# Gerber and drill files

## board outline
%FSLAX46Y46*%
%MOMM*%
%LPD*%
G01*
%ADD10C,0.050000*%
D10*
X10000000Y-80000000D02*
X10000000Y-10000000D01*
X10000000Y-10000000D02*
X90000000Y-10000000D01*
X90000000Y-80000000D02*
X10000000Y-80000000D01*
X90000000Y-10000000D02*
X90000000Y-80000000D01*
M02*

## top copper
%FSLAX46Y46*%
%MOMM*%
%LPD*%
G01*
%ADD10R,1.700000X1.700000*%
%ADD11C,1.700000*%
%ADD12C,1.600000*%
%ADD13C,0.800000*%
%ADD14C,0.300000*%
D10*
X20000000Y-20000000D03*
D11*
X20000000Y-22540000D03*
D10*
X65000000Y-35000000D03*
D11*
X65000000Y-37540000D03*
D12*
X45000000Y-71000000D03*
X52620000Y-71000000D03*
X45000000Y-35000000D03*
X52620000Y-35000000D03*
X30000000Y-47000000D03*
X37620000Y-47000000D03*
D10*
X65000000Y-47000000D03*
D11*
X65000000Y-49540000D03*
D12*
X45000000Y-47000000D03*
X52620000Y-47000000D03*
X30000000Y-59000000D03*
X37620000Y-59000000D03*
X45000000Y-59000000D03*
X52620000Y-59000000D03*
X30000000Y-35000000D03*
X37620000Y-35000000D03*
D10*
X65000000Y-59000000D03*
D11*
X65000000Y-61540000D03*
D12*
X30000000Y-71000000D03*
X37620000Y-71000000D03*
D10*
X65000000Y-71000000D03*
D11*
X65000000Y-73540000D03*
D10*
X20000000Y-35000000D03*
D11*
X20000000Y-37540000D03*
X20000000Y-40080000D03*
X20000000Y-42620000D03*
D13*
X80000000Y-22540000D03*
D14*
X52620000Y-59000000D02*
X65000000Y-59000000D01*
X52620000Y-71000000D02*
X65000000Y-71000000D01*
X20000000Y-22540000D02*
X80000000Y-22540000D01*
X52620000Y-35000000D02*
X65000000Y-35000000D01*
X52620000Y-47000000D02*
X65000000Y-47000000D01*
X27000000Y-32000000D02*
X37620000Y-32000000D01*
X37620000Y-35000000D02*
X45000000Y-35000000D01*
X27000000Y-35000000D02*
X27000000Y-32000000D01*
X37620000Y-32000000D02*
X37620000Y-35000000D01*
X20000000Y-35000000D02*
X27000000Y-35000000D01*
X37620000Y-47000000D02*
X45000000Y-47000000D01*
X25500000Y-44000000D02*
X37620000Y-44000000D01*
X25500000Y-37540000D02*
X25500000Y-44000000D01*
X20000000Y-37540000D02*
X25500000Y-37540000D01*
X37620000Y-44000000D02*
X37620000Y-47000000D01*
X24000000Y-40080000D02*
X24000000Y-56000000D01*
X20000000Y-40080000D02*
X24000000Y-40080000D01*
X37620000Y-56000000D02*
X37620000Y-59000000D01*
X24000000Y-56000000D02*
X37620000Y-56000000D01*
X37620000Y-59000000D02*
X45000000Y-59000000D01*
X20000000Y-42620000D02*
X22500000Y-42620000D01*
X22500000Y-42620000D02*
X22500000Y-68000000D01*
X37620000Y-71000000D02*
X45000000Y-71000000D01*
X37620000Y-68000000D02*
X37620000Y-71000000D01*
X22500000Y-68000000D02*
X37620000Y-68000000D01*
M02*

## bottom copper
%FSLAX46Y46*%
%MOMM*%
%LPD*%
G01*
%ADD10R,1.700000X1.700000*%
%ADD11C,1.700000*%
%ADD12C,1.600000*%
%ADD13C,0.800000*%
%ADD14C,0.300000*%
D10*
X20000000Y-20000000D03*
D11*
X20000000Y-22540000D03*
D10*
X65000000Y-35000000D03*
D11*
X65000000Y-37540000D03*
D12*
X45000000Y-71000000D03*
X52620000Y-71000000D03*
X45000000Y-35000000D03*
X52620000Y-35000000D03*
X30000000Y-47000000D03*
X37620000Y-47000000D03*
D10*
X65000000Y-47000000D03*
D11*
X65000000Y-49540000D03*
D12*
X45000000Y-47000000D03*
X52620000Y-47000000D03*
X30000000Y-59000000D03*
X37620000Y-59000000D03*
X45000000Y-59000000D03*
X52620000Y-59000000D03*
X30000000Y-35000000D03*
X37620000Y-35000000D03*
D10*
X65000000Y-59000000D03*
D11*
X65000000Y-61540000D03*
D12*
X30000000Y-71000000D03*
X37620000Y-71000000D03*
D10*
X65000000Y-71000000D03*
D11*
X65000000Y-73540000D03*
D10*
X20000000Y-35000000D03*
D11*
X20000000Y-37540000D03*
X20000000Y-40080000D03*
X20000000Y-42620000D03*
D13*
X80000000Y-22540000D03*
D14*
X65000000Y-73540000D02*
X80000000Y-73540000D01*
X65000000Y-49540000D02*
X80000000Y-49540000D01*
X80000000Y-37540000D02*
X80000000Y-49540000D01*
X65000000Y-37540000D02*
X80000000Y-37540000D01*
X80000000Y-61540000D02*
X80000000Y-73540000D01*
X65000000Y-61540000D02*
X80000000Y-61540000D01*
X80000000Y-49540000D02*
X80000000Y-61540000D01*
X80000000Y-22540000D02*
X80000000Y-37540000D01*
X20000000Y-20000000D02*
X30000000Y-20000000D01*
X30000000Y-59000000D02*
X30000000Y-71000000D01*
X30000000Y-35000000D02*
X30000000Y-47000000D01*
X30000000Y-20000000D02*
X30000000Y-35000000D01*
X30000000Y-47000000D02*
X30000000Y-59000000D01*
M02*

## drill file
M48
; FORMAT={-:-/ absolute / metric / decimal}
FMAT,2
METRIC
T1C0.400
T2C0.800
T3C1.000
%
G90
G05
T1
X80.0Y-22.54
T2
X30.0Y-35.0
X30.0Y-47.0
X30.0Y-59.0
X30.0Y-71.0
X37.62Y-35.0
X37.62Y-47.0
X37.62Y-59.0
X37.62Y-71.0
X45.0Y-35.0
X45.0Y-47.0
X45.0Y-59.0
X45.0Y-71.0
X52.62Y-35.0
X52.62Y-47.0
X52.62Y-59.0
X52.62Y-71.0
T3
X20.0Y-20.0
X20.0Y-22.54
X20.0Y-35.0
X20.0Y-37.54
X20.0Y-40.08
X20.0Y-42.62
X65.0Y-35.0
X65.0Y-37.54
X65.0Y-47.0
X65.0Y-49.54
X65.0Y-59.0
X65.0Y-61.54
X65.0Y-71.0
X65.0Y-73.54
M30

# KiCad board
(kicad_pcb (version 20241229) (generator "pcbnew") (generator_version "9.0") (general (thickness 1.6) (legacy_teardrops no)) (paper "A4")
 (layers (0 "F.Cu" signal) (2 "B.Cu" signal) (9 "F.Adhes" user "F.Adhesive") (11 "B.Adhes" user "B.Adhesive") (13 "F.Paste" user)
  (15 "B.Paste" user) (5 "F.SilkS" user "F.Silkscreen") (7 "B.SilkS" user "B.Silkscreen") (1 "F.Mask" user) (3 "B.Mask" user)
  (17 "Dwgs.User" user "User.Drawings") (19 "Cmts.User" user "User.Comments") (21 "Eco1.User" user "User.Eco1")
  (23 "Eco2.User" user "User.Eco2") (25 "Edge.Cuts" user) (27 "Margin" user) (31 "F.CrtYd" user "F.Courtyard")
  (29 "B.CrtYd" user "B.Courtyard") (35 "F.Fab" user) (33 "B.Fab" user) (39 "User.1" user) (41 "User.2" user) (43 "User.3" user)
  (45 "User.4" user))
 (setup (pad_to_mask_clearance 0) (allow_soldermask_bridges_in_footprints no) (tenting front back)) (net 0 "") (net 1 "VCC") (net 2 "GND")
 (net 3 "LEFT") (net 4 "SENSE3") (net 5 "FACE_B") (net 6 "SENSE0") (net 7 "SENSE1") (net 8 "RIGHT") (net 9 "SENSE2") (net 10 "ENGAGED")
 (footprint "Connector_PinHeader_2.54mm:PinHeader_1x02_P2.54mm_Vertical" (layer "F.Cu") (at 20 20)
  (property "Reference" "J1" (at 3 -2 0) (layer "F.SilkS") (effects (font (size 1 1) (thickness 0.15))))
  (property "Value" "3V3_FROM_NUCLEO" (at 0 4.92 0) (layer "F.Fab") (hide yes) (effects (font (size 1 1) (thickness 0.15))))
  (pad "1" thru_hole rect (at 0 0) (size 1.7 1.7) (drill 1) (layers "*.Cu" "*.Mask") (remove_unused_layers no) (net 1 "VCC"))
  (pad "2" thru_hole circle (at 0 2.54) (size 1.7 1.7) (drill 1) (layers "*.Cu" "*.Mask") (remove_unused_layers no) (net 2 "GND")))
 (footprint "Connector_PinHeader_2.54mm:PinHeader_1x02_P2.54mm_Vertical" (layer "F.Cu") (at 65 35)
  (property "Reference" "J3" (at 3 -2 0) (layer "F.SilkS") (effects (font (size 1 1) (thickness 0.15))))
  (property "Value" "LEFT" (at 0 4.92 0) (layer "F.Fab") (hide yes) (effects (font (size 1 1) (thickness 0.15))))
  (pad "1" thru_hole rect (at 0 0) (size 1.7 1.7) (drill 1) (layers "*.Cu" "*.Mask") (remove_unused_layers no) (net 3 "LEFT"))
  (pad "2" thru_hole circle (at 0 2.54) (size 1.7 1.7) (drill 1) (layers "*.Cu" "*.Mask") (remove_unused_layers no) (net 2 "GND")))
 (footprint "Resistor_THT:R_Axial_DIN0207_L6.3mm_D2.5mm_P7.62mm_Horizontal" (layer "F.Cu") (at 45 71)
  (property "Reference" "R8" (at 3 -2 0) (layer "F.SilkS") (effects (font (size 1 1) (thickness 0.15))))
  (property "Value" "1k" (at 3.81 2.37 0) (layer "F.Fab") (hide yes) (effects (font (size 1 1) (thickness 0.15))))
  (pad "1" thru_hole circle (at 0 0) (size 1.6 1.6) (drill 0.8) (layers "*.Cu" "*.Mask") (remove_unused_layers no) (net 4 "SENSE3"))
  (pad "2" thru_hole circle (at 7.62 0) (size 1.6 1.6) (drill 0.8) (layers "*.Cu" "*.Mask") (remove_unused_layers no) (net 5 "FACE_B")))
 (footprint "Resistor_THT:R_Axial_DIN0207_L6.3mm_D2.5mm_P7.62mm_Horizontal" (layer "F.Cu") (at 45 35)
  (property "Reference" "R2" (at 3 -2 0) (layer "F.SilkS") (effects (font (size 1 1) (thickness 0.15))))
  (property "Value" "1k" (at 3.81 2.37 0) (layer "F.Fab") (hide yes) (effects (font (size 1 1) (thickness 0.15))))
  (pad "1" thru_hole circle (at 0 0) (size 1.6 1.6) (drill 0.8) (layers "*.Cu" "*.Mask") (remove_unused_layers no) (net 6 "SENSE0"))
  (pad "2" thru_hole circle (at 7.62 0) (size 1.6 1.6) (drill 0.8) (layers "*.Cu" "*.Mask") (remove_unused_layers no) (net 3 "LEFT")))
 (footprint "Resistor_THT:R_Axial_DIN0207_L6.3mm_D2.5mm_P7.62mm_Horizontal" (layer "F.Cu") (at 30 47)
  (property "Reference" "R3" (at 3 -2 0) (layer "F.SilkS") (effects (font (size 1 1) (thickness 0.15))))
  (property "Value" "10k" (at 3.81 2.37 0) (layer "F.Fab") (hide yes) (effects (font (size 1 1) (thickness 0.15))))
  (pad "1" thru_hole circle (at 0 0) (size 1.6 1.6) (drill 0.8) (layers "*.Cu" "*.Mask") (remove_unused_layers no) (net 1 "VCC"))
  (pad "2" thru_hole circle (at 7.62 0) (size 1.6 1.6) (drill 0.8) (layers "*.Cu" "*.Mask") (remove_unused_layers no) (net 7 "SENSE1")))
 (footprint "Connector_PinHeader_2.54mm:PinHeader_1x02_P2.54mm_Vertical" (layer "F.Cu") (at 65 47)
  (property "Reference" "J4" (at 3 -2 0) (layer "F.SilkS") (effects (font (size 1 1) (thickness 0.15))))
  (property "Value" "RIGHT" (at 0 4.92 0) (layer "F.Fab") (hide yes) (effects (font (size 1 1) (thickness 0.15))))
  (pad "1" thru_hole rect (at 0 0) (size 1.7 1.7) (drill 1) (layers "*.Cu" "*.Mask") (remove_unused_layers no) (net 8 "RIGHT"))
  (pad "2" thru_hole circle (at 0 2.54) (size 1.7 1.7) (drill 1) (layers "*.Cu" "*.Mask") (remove_unused_layers no) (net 2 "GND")))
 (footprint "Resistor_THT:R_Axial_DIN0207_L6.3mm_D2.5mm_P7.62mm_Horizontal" (layer "F.Cu") (at 45 47)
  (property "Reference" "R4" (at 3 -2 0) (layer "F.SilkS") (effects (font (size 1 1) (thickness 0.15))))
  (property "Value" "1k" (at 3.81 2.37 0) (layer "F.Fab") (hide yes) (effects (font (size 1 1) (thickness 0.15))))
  (pad "1" thru_hole circle (at 0 0) (size 1.6 1.6) (drill 0.8) (layers "*.Cu" "*.Mask") (remove_unused_layers no) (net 7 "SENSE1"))
  (pad "2" thru_hole circle (at 7.62 0) (size 1.6 1.6) (drill 0.8) (layers "*.Cu" "*.Mask") (remove_unused_layers no) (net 8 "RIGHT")))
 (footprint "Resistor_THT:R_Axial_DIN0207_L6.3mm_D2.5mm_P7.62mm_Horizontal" (layer "F.Cu") (at 30 59)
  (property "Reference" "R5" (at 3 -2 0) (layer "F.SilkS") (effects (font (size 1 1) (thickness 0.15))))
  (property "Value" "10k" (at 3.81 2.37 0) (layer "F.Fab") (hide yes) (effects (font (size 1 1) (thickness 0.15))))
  (pad "1" thru_hole circle (at 0 0) (size 1.6 1.6) (drill 0.8) (layers "*.Cu" "*.Mask") (remove_unused_layers no) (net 1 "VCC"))
  (pad "2" thru_hole circle (at 7.62 0) (size 1.6 1.6) (drill 0.8) (layers "*.Cu" "*.Mask") (remove_unused_layers no) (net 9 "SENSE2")))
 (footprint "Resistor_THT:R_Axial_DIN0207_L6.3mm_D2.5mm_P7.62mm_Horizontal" (layer "F.Cu") (at 45 59)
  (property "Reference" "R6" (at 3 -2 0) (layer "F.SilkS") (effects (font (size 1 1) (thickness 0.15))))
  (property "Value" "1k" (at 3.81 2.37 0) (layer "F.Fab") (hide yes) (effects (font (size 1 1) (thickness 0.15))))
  (pad "1" thru_hole circle (at 0 0) (size 1.6 1.6) (drill 0.8) (layers "*.Cu" "*.Mask") (remove_unused_layers no) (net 9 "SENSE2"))
  (pad "2" thru_hole circle (at 7.62 0) (size 1.6 1.6) (drill 0.8) (layers "*.Cu" "*.Mask") (remove_unused_layers no) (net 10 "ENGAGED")))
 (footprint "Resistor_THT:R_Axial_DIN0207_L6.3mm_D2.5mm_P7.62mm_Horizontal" (layer "F.Cu") (at 30 35)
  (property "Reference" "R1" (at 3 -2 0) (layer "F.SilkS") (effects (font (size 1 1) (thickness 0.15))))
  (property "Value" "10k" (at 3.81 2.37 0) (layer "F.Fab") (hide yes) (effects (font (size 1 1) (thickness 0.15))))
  (pad "1" thru_hole circle (at 0 0) (size 1.6 1.6) (drill 0.8) (layers "*.Cu" "*.Mask") (remove_unused_layers no) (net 1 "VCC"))
  (pad "2" thru_hole circle (at 7.62 0) (size 1.6 1.6) (drill 0.8) (layers "*.Cu" "*.Mask") (remove_unused_layers no) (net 6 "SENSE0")))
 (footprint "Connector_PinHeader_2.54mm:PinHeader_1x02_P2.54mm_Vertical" (layer "F.Cu") (at 65 59)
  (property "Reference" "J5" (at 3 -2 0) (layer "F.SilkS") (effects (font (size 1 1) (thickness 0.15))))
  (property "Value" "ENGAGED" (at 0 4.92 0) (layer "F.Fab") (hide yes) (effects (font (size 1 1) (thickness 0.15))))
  (pad "1" thru_hole rect (at 0 0) (size 1.7 1.7) (drill 1) (layers "*.Cu" "*.Mask") (remove_unused_layers no) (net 10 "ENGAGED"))
  (pad "2" thru_hole circle (at 0 2.54) (size 1.7 1.7) (drill 1) (layers "*.Cu" "*.Mask") (remove_unused_layers no) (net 2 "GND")))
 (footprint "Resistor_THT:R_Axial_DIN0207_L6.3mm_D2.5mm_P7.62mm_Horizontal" (layer "F.Cu") (at 30 71)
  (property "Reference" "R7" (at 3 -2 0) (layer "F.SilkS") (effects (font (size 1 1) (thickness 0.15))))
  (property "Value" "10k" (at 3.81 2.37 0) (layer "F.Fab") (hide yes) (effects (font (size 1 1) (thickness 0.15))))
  (pad "1" thru_hole circle (at 0 0) (size 1.6 1.6) (drill 0.8) (layers "*.Cu" "*.Mask") (remove_unused_layers no) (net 1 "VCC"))
  (pad "2" thru_hole circle (at 7.62 0) (size 1.6 1.6) (drill 0.8) (layers "*.Cu" "*.Mask") (remove_unused_layers no) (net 4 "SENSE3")))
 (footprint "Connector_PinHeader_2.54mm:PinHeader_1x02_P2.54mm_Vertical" (layer "F.Cu") (at 65 71)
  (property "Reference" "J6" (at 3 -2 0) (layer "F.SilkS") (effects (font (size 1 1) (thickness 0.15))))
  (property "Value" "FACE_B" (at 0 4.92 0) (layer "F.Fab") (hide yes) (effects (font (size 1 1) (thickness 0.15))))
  (pad "1" thru_hole rect (at 0 0) (size 1.7 1.7) (drill 1) (layers "*.Cu" "*.Mask") (remove_unused_layers no) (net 5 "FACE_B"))
  (pad "2" thru_hole circle (at 0 2.54) (size 1.7 1.7) (drill 1) (layers "*.Cu" "*.Mask") (remove_unused_layers no) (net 2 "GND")))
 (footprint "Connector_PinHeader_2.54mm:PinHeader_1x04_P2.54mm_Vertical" (layer "F.Cu") (at 20 35)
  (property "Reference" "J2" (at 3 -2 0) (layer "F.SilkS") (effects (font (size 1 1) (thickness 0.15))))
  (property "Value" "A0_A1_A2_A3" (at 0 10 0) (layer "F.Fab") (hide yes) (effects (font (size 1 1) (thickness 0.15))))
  (pad "1" thru_hole rect (at 0 0) (size 1.7 1.7) (drill 1) (layers "*.Cu" "*.Mask") (remove_unused_layers no) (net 6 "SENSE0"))
  (pad "2" thru_hole circle (at 0 2.54) (size 1.7 1.7) (drill 1) (layers "*.Cu" "*.Mask") (remove_unused_layers no) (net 7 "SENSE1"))
  (pad "3" thru_hole circle (at 0 5.08) (size 1.7 1.7) (drill 1) (layers "*.Cu" "*.Mask") (remove_unused_layers no) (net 9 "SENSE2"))
  (pad "4" thru_hole circle (at 0 7.62) (size 1.7 1.7) (drill 1) (layers "*.Cu" "*.Mask") (remove_unused_layers no) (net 4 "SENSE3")))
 (gr_line (start 10 80) (end 10 10) (stroke (width 0.05) (type default)) (layer "Edge.Cuts"))
 (gr_line (start 10 10) (end 90 10) (stroke (width 0.05) (type default)) (layer "Edge.Cuts"))
 (gr_line (start 90 80) (end 10 80) (stroke (width 0.05) (type default)) (layer "Edge.Cuts"))
 (gr_line (start 90 10) (end 90 80) (stroke (width 0.05) (type default)) (layer "Edge.Cuts"))
 (segment (start 52.62 59) (end 65 59) (width 0.3) (layer "F.Cu") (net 10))
 (segment (start 52.62 71) (end 65 71) (width 0.3) (layer "F.Cu") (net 5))
 (segment (start 20 22.54) (end 80 22.54) (width 0.3) (layer "F.Cu") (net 2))
 (via (at 80 22.54) (size 0.8) (drill 0.4) (layers "F.Cu" "B.Cu") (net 2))
 (segment (start 65 73.54) (end 80 73.54) (width 0.3) (layer "B.Cu") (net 2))
 (segment (start 65 49.54) (end 80 49.54) (width 0.3) (layer "B.Cu") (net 2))
 (segment (start 80 37.54) (end 80 49.54) (width 0.3) (layer "B.Cu") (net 2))
 (segment (start 65 37.54) (end 80 37.54) (width 0.3) (layer "B.Cu") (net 2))
 (segment (start 80 61.54) (end 80 73.54) (width 0.3) (layer "B.Cu") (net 2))
 (segment (start 65 61.54) (end 80 61.54) (width 0.3) (layer "B.Cu") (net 2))
 (segment (start 80 49.54) (end 80 61.54) (width 0.3) (layer "B.Cu") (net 2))
 (segment (start 80 22.54) (end 80 37.54) (width 0.3) (layer "B.Cu") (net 2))
 (segment (start 52.62 35) (end 65 35) (width 0.3) (layer "F.Cu") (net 3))
 (segment (start 52.62 47) (end 65 47) (width 0.3) (layer "F.Cu") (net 8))
 (segment (start 27 32) (end 37.62 32) (width 0.3) (layer "F.Cu") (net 6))
 (segment (start 37.62 35) (end 45 35) (width 0.3) (layer "F.Cu") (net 6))
 (segment (start 27 35) (end 27 32) (width 0.3) (layer "F.Cu") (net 6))
 (segment (start 37.62 32) (end 37.62 35) (width 0.3) (layer "F.Cu") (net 6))
 (segment (start 20 35) (end 27 35) (width 0.3) (layer "F.Cu") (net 6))
 (segment (start 37.62 47) (end 45 47) (width 0.3) (layer "F.Cu") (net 7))
 (segment (start 25.5 44) (end 37.62 44) (width 0.3) (layer "F.Cu") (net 7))
 (segment (start 25.5 37.54) (end 25.5 44) (width 0.3) (layer "F.Cu") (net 7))
 (segment (start 20 37.54) (end 25.5 37.54) (width 0.3) (layer "F.Cu") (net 7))
 (segment (start 37.62 44) (end 37.62 47) (width 0.3) (layer "F.Cu") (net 7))
 (segment (start 24 40.08) (end 24 56) (width 0.3) (layer "F.Cu") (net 9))
 (segment (start 20 40.08) (end 24 40.08) (width 0.3) (layer "F.Cu") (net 9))
 (segment (start 37.62 56) (end 37.62 59) (width 0.3) (layer "F.Cu") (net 9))
 (segment (start 24 56) (end 37.62 56) (width 0.3) (layer "F.Cu") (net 9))
 (segment (start 37.62 59) (end 45 59) (width 0.3) (layer "F.Cu") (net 9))
 (segment (start 20 42.62) (end 22.5 42.62) (width 0.3) (layer "F.Cu") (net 4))
 (segment (start 22.5 42.62) (end 22.5 68) (width 0.3) (layer "F.Cu") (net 4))
 (segment (start 37.62 71) (end 45 71) (width 0.3) (layer "F.Cu") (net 4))
 (segment (start 37.62 68) (end 37.62 71) (width 0.3) (layer "F.Cu") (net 4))
 (segment (start 22.5 68) (end 37.62 68) (width 0.3) (layer "F.Cu") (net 4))
 (segment (start 20 20) (end 30 20) (width 0.3) (layer "B.Cu") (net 1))
 (segment (start 30 59) (end 30 71) (width 0.3) (layer "B.Cu") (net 1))
 (segment (start 30 35) (end 30 47) (width 0.3) (layer "B.Cu") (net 1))
 (segment (start 30 20) (end 30 35) (width 0.3) (layer "B.Cu") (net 1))
 (segment (start 30 47) (end 30 59) (width 0.3) (layer "B.Cu") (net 1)))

